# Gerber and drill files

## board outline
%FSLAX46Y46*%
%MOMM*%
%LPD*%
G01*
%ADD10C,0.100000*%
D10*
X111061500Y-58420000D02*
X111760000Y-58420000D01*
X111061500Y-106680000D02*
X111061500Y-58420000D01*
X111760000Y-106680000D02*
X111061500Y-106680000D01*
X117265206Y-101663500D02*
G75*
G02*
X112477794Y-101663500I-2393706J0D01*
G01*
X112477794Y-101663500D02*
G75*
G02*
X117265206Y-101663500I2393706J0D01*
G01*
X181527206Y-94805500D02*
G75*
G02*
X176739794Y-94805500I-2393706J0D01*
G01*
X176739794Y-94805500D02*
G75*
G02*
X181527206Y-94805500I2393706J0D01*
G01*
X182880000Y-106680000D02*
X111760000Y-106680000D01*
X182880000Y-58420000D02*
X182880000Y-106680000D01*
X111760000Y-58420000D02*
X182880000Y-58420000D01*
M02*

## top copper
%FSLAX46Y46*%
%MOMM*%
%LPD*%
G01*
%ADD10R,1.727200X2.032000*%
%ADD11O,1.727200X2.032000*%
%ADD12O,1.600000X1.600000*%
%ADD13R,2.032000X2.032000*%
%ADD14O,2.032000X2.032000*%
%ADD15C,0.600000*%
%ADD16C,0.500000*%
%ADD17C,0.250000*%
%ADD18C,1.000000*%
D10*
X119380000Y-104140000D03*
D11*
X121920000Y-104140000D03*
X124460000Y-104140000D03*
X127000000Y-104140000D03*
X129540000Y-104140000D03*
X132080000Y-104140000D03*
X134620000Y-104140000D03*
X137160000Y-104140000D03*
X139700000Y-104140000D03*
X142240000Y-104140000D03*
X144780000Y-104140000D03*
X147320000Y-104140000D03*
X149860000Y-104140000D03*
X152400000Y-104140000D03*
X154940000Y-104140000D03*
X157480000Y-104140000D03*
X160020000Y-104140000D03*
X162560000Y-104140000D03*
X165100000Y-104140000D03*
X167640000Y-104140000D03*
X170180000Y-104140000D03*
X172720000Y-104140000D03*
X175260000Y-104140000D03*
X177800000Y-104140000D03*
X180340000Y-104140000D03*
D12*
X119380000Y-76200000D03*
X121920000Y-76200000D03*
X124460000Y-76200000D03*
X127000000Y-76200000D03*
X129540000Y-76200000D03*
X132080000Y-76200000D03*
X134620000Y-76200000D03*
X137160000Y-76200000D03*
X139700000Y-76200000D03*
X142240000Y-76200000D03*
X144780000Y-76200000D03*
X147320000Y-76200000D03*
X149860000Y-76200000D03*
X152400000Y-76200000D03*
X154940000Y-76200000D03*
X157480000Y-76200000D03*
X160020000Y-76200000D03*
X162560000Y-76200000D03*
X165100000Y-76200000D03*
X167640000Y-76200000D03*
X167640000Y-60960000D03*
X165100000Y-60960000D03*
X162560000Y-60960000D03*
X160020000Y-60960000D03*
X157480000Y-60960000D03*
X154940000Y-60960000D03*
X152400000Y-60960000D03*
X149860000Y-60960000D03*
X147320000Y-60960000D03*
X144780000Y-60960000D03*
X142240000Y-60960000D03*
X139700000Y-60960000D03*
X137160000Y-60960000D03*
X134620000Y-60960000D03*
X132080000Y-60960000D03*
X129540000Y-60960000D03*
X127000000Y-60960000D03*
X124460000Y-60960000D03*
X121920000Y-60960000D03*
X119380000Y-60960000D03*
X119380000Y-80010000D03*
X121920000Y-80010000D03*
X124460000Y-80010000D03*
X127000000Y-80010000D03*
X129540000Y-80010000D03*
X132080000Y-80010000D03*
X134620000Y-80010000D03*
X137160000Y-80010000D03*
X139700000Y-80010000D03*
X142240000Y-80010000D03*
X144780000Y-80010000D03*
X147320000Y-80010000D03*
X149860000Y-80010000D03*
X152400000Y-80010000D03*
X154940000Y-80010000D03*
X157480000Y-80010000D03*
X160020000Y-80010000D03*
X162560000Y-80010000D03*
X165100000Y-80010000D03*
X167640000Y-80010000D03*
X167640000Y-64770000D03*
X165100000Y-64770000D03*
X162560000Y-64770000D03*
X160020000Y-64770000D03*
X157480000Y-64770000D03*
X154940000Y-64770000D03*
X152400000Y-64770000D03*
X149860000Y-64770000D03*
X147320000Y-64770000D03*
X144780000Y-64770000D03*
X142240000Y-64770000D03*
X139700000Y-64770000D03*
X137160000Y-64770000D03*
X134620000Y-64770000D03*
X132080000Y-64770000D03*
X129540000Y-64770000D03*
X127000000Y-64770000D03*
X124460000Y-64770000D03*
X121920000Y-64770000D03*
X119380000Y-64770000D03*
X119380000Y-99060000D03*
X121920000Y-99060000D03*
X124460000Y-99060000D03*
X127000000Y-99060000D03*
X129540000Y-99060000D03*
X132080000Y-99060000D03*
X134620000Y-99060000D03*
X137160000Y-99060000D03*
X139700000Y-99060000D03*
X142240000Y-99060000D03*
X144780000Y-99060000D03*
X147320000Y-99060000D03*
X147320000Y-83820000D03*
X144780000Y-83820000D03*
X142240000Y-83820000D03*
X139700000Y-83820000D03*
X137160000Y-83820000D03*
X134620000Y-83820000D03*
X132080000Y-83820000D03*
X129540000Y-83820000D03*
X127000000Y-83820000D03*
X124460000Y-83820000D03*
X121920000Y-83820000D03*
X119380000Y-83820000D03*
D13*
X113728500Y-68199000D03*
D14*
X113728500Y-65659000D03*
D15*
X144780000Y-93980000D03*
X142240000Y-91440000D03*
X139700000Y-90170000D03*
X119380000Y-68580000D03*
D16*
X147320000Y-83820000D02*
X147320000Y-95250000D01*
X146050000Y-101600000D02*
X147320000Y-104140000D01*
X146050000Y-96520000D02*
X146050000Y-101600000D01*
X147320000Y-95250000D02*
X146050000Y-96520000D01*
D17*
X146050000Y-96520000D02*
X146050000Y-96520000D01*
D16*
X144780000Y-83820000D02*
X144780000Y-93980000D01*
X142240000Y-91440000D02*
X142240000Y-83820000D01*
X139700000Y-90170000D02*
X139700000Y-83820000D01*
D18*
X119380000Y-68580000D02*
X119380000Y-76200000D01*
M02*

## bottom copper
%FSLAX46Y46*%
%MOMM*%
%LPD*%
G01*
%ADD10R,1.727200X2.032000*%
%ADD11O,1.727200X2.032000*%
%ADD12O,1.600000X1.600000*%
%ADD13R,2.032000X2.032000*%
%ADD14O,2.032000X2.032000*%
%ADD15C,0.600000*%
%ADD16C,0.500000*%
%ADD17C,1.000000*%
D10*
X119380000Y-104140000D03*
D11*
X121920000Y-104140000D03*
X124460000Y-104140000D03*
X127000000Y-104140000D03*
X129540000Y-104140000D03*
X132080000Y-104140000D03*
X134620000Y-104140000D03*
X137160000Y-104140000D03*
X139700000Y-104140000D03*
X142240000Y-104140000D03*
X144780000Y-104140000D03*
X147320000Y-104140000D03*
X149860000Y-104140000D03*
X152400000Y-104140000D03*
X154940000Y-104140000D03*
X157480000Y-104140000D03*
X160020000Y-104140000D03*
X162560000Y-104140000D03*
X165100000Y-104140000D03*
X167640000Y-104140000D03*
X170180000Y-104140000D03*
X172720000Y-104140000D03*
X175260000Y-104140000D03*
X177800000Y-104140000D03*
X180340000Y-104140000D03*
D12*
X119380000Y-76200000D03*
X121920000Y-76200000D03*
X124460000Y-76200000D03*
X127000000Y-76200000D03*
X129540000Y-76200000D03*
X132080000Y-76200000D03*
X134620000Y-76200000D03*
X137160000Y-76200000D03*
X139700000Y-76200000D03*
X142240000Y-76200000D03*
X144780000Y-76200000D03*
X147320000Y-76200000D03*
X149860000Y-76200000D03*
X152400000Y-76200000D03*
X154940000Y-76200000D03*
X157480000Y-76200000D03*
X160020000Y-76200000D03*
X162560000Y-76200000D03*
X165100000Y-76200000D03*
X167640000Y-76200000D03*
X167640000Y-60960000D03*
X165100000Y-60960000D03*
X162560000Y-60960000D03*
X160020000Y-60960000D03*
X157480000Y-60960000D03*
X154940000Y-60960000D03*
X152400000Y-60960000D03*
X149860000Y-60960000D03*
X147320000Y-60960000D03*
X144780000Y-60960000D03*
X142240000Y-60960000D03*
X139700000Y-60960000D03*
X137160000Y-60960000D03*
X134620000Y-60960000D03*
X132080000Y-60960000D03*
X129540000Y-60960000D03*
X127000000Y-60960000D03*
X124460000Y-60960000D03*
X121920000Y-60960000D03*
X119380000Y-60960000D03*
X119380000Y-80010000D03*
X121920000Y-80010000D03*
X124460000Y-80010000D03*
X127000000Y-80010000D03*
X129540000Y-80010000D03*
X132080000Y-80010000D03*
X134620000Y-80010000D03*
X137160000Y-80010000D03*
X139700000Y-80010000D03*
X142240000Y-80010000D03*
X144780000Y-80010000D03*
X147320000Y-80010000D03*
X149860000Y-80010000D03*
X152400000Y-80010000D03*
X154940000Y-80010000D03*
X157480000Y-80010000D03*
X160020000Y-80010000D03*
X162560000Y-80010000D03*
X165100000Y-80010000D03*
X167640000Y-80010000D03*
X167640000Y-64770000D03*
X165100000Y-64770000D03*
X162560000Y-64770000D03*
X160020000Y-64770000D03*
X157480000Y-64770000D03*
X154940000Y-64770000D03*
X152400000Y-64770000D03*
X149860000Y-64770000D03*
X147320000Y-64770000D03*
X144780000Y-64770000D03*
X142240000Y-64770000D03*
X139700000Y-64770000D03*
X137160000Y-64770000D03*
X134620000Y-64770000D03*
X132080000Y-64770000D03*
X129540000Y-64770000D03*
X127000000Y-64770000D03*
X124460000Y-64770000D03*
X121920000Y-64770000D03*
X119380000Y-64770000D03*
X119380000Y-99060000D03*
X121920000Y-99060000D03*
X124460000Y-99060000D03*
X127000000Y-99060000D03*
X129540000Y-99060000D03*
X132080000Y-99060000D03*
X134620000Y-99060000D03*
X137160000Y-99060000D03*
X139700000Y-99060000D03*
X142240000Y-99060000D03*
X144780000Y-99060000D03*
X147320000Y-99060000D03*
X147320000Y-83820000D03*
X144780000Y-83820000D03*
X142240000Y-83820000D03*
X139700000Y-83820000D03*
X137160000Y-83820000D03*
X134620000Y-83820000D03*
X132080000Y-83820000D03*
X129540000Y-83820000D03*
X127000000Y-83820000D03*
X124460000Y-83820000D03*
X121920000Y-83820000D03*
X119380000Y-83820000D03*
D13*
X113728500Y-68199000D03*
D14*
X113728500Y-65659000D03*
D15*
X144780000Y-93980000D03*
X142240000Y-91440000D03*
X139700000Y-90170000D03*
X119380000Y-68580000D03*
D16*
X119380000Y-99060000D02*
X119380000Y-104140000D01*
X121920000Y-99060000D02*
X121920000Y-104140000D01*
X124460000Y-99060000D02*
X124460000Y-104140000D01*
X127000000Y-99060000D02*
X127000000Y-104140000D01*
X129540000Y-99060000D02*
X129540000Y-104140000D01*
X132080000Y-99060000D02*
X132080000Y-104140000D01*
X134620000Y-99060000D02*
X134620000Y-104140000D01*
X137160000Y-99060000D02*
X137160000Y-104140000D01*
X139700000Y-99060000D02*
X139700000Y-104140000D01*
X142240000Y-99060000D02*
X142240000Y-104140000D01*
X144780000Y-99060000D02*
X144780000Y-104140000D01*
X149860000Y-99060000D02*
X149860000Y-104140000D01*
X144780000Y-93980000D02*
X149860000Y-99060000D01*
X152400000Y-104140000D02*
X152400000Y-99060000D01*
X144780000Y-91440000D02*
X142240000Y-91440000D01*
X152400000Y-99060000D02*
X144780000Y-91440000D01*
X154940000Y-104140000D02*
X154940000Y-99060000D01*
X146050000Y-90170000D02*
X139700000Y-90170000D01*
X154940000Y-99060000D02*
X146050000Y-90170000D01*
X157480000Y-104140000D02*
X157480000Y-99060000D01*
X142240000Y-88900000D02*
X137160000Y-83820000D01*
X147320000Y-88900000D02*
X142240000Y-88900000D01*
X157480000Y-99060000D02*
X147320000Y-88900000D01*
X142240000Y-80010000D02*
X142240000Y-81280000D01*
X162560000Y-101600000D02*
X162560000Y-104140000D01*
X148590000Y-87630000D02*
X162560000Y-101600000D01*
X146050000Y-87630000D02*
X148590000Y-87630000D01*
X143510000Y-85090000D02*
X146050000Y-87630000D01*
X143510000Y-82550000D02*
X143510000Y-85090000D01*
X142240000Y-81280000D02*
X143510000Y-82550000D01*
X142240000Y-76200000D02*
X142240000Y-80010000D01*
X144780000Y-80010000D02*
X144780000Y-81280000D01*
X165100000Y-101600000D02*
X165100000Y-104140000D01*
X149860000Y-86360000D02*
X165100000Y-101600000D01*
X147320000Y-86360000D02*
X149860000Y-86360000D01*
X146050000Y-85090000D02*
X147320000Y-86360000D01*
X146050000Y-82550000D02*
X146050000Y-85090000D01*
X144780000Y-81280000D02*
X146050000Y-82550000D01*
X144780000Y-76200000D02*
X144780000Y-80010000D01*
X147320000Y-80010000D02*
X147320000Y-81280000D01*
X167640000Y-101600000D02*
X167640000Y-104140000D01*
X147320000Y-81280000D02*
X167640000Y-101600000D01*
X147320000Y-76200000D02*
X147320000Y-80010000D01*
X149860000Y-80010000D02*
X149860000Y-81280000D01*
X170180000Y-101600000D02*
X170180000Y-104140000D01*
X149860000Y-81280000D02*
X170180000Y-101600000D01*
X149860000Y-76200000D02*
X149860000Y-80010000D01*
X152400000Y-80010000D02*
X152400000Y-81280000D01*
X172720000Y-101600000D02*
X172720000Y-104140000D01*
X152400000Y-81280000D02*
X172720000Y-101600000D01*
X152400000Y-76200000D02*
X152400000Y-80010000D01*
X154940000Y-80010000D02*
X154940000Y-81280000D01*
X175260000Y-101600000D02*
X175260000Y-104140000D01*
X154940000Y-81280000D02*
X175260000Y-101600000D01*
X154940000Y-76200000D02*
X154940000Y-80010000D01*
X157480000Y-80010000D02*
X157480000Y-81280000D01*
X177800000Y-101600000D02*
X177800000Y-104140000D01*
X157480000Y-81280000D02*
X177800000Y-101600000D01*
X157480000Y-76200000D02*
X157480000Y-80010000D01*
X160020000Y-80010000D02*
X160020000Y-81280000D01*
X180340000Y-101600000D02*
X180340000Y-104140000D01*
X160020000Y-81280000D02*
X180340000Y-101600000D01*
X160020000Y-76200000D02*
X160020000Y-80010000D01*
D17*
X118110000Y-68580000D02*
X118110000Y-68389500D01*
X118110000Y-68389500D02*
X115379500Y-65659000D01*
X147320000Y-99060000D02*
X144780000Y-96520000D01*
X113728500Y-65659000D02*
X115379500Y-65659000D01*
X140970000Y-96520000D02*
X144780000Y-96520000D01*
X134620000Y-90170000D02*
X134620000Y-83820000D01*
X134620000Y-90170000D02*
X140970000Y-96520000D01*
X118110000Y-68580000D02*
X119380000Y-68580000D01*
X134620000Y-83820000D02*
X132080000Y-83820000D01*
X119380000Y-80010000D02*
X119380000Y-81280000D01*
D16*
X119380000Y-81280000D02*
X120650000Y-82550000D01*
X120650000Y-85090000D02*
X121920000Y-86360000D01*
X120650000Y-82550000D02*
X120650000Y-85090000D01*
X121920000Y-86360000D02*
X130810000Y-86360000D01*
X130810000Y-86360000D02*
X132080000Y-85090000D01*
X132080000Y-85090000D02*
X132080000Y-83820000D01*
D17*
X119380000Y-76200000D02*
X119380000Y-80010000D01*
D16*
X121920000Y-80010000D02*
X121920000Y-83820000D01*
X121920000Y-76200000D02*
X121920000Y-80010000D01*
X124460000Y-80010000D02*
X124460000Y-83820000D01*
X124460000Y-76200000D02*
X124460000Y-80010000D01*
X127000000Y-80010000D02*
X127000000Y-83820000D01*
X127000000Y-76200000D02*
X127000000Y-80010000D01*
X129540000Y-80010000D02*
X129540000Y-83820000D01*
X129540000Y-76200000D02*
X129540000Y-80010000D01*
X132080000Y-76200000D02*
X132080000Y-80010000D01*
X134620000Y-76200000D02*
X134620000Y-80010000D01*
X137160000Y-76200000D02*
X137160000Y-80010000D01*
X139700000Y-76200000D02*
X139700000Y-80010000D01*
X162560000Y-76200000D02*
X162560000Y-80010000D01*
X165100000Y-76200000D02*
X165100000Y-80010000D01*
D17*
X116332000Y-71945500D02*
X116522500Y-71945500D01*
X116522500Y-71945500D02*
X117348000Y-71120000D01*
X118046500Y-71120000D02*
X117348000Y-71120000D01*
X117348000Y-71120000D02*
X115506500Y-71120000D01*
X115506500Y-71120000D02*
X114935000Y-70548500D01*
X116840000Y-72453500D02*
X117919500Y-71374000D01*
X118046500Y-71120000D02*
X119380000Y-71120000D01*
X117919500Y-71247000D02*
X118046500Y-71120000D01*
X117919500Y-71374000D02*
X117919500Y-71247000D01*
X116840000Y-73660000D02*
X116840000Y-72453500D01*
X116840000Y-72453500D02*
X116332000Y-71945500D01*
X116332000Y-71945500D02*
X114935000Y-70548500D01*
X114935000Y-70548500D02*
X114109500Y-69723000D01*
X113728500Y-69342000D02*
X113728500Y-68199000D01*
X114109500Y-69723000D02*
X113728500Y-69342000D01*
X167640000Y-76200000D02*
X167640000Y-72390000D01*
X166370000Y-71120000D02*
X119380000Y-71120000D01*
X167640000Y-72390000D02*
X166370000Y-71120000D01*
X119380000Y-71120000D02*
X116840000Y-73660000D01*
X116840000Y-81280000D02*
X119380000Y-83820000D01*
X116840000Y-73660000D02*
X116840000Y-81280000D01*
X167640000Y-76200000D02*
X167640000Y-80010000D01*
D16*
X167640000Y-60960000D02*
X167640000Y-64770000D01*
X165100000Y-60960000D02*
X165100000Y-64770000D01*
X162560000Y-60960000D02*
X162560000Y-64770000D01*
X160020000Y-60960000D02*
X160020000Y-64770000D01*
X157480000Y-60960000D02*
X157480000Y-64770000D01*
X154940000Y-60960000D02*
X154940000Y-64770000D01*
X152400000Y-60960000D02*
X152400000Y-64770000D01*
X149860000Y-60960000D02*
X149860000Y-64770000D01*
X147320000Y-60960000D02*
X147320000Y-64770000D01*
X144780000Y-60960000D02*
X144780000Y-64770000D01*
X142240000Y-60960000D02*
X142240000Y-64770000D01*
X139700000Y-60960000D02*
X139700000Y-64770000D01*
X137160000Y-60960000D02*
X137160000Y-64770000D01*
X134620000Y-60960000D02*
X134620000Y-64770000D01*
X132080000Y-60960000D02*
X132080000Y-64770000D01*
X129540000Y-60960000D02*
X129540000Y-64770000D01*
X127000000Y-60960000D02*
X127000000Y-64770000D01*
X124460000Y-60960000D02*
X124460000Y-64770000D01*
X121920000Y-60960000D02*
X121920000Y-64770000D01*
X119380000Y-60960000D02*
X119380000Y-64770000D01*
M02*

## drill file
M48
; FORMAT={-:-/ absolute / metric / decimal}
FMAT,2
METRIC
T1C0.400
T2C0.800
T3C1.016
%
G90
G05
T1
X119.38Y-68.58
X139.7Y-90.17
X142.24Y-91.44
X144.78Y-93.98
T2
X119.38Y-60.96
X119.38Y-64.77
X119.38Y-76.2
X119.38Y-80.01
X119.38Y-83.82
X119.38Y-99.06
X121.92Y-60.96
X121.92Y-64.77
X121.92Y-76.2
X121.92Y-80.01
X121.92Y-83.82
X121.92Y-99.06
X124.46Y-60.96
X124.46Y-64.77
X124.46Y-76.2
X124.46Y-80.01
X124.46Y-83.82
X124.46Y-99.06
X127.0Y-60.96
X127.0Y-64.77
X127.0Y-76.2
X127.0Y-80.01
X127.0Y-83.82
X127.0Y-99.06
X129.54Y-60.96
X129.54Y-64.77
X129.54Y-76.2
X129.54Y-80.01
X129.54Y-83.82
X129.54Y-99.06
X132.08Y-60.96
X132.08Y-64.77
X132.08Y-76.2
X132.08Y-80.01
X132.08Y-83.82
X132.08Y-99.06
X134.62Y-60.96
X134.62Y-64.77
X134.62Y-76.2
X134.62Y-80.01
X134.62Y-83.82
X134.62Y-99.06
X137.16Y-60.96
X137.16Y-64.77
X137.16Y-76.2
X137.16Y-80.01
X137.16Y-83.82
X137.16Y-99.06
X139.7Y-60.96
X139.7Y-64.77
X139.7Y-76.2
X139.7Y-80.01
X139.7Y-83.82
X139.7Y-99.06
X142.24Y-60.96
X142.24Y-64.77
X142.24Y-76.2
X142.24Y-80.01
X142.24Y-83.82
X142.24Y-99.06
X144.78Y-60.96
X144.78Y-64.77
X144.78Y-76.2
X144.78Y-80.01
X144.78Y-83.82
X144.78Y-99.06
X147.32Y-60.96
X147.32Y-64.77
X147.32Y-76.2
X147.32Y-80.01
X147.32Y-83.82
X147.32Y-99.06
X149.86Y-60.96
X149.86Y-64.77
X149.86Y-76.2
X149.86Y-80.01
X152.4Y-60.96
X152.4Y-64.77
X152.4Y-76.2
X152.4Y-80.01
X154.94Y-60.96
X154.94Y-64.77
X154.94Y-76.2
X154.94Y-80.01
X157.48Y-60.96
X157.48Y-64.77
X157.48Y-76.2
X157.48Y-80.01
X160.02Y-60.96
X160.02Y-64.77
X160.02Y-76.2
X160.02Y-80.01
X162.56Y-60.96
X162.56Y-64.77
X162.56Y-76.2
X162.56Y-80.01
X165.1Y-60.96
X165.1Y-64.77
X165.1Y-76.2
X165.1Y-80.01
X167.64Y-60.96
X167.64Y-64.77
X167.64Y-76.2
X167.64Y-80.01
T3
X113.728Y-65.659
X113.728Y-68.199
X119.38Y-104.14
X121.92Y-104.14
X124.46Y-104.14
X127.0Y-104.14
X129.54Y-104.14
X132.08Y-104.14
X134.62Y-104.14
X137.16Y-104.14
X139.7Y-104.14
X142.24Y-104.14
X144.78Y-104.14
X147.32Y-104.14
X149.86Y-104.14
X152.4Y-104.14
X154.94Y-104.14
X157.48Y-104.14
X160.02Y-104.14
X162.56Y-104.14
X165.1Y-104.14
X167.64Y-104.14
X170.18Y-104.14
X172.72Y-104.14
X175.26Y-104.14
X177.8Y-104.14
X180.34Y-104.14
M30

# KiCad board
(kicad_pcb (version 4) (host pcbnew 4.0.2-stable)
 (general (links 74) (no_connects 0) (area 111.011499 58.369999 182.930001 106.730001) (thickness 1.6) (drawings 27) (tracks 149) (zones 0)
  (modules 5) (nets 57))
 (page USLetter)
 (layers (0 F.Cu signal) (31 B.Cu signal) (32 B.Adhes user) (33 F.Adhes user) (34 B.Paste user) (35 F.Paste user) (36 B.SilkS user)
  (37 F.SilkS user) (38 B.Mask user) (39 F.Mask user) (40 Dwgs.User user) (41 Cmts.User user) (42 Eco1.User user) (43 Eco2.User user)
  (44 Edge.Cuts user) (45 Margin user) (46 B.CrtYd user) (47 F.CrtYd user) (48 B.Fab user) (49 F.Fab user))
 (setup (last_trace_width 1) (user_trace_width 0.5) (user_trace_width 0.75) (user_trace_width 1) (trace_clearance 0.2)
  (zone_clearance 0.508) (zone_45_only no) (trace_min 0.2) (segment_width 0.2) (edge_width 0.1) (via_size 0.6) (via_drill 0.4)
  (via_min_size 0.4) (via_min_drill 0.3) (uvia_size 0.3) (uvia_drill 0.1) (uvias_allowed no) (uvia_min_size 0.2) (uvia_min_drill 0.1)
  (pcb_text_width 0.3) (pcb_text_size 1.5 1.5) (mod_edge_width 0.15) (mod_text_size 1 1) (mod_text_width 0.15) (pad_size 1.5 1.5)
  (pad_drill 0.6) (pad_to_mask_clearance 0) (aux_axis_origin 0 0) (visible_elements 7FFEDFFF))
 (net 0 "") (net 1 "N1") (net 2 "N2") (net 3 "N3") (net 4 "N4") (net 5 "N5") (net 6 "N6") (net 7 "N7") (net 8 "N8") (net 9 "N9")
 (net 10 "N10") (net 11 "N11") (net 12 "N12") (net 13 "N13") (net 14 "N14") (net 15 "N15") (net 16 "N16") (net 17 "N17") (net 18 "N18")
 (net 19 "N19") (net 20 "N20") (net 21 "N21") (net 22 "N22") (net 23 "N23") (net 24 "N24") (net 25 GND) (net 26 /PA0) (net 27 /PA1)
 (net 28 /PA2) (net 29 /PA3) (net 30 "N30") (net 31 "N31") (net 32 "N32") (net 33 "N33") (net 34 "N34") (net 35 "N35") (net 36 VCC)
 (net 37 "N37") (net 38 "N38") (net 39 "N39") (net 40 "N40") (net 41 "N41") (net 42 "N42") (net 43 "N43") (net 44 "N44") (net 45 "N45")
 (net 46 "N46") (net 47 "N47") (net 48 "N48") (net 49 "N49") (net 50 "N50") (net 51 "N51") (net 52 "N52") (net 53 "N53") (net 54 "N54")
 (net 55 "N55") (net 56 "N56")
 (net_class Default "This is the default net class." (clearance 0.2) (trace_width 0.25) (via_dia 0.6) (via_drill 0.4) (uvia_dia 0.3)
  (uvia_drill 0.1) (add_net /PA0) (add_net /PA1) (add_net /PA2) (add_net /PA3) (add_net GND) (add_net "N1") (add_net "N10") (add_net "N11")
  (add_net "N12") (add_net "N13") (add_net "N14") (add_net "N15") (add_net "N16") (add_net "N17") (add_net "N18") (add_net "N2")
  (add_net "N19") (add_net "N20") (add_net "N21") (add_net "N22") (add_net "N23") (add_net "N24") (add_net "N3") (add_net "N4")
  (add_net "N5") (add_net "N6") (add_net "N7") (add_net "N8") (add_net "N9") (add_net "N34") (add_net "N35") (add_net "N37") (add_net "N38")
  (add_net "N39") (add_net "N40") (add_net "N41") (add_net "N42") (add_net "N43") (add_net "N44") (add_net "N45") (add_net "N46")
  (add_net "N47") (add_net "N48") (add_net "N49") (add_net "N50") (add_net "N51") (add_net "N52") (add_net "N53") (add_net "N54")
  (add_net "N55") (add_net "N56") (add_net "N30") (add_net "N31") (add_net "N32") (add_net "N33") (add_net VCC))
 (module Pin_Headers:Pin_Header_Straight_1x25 (layer F.Cu) (at 119.38 104.14 90)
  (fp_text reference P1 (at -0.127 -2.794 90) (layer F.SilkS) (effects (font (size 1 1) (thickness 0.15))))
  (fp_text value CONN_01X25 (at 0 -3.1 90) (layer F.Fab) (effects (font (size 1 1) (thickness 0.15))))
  (pad 1 thru_hole rect (at 0 0 90) (size 2.032 1.7272) (drill 1.016) (layers *.Cu *.Mask F.SilkS) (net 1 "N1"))
  (pad 2 thru_hole oval (at 0 2.54 90) (size 2.032 1.7272) (drill 1.016) (layers *.Cu *.Mask F.SilkS) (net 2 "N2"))
  (pad 3 thru_hole oval (at 0 5.08 90) (size 2.032 1.7272) (drill 1.016) (layers *.Cu *.Mask F.SilkS) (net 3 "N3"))
  (pad 4 thru_hole oval (at 0 7.62 90) (size 2.032 1.7272) (drill 1.016) (layers *.Cu *.Mask F.SilkS) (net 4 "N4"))
  (pad 5 thru_hole oval (at 0 10.16 90) (size 2.032 1.7272) (drill 1.016) (layers *.Cu *.Mask F.SilkS) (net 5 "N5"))
  (pad 6 thru_hole oval (at 0 12.7 90) (size 2.032 1.7272) (drill 1.016) (layers *.Cu *.Mask F.SilkS) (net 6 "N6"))
  (pad 7 thru_hole oval (at 0 15.24 90) (size 2.032 1.7272) (drill 1.016) (layers *.Cu *.Mask F.SilkS) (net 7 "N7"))
  (pad 8 thru_hole oval (at 0 17.78 90) (size 2.032 1.7272) (drill 1.016) (layers *.Cu *.Mask F.SilkS) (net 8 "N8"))
  (pad 9 thru_hole oval (at 0 20.32 90) (size 2.032 1.7272) (drill 1.016) (layers *.Cu *.Mask F.SilkS) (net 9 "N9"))
  (pad 10 thru_hole oval (at 0 22.86 90) (size 2.032 1.7272) (drill 1.016) (layers *.Cu *.Mask F.SilkS) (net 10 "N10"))
  (pad 11 thru_hole oval (at 0 25.4 90) (size 2.032 1.7272) (drill 1.016) (layers *.Cu *.Mask F.SilkS) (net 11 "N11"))
  (pad 12 thru_hole oval (at 0 27.94 90) (size 2.032 1.7272) (drill 1.016) (layers *.Cu *.Mask F.SilkS) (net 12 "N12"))
  (pad 13 thru_hole oval (at 0 30.48 90) (size 2.032 1.7272) (drill 1.016) (layers *.Cu *.Mask F.SilkS) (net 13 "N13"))
  (pad 14 thru_hole oval (at 0 33.02 90) (size 2.032 1.7272) (drill 1.016) (layers *.Cu *.Mask F.SilkS) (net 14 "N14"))
  (pad 15 thru_hole oval (at 0 35.56 90) (size 2.032 1.7272) (drill 1.016) (layers *.Cu *.Mask F.SilkS) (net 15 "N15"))
  (pad 16 thru_hole oval (at 0 38.1 90) (size 2.032 1.7272) (drill 1.016) (layers *.Cu *.Mask F.SilkS) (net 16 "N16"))
  (pad 17 thru_hole oval (at 0 40.64 90) (size 2.032 1.7272) (drill 1.016) (layers *.Cu *.Mask F.SilkS))
  (pad 18 thru_hole oval (at 0 43.18 90) (size 2.032 1.7272) (drill 1.016) (layers *.Cu *.Mask F.SilkS) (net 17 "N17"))
  (pad 19 thru_hole oval (at 0 45.72 90) (size 2.032 1.7272) (drill 1.016) (layers *.Cu *.Mask F.SilkS) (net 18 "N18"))
  (pad 20 thru_hole oval (at 0 48.26 90) (size 2.032 1.7272) (drill 1.016) (layers *.Cu *.Mask F.SilkS) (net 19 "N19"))
  (pad 21 thru_hole oval (at 0 50.8 90) (size 2.032 1.7272) (drill 1.016) (layers *.Cu *.Mask F.SilkS) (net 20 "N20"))
  (pad 22 thru_hole oval (at 0 53.34 90) (size 2.032 1.7272) (drill 1.016) (layers *.Cu *.Mask F.SilkS) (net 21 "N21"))
  (pad 23 thru_hole oval (at 0 55.88 90) (size 2.032 1.7272) (drill 1.016) (layers *.Cu *.Mask F.SilkS) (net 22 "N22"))
  (pad 24 thru_hole oval (at 0 58.42 90) (size 2.032 1.7272) (drill 1.016) (layers *.Cu *.Mask F.SilkS) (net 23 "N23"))
  (pad 25 thru_hole oval (at 0 60.96 90) (size 2.032 1.7272) (drill 1.016) (layers *.Cu *.Mask F.SilkS) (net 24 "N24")))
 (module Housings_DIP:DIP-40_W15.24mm (layer F.Cu) (at 119.38 76.2 90)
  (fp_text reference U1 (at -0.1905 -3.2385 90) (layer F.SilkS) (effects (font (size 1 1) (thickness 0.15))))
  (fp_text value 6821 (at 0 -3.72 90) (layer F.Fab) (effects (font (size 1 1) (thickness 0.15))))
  (pad 1 thru_hole oval (at 0 0 90) (size 1.6 1.6) (drill 0.8) (layers *.Cu *.Mask F.SilkS) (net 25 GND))
  (pad 2 thru_hole oval (at 0 2.54 90) (size 1.6 1.6) (drill 0.8) (layers *.Cu *.Mask F.SilkS) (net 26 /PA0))
  (pad 3 thru_hole oval (at 0 5.08 90) (size 1.6 1.6) (drill 0.8) (layers *.Cu *.Mask F.SilkS) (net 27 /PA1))
  (pad 4 thru_hole oval (at 0 7.62 90) (size 1.6 1.6) (drill 0.8) (layers *.Cu *.Mask F.SilkS) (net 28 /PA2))
  (pad 5 thru_hole oval (at 0 10.16 90) (size 1.6 1.6) (drill 0.8) (layers *.Cu *.Mask F.SilkS) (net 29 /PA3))
  (pad 6 thru_hole oval (at 0 12.7 90) (size 1.6 1.6) (drill 0.8) (layers *.Cu *.Mask F.SilkS) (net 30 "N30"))
  (pad 7 thru_hole oval (at 0 15.24 90) (size 1.6 1.6) (drill 0.8) (layers *.Cu *.Mask F.SilkS) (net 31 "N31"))
  (pad 8 thru_hole oval (at 0 17.78 90) (size 1.6 1.6) (drill 0.8) (layers *.Cu *.Mask F.SilkS) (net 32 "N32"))
  (pad 9 thru_hole oval (at 0 20.32 90) (size 1.6 1.6) (drill 0.8) (layers *.Cu *.Mask F.SilkS) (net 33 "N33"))
  (pad 10 thru_hole oval (at 0 22.86 90) (size 1.6 1.6) (drill 0.8) (layers *.Cu *.Mask F.SilkS) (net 17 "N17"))
  (pad 11 thru_hole oval (at 0 25.4 90) (size 1.6 1.6) (drill 0.8) (layers *.Cu *.Mask F.SilkS) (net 18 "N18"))
  (pad 12 thru_hole oval (at 0 27.94 90) (size 1.6 1.6) (drill 0.8) (layers *.Cu *.Mask F.SilkS) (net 19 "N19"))
  (pad 13 thru_hole oval (at 0 30.48 90) (size 1.6 1.6) (drill 0.8) (layers *.Cu *.Mask F.SilkS) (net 20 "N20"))
  (pad 14 thru_hole oval (at 0 33.02 90) (size 1.6 1.6) (drill 0.8) (layers *.Cu *.Mask F.SilkS) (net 21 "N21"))
  (pad 15 thru_hole oval (at 0 35.56 90) (size 1.6 1.6) (drill 0.8) (layers *.Cu *.Mask F.SilkS) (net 22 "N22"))
  (pad 16 thru_hole oval (at 0 38.1 90) (size 1.6 1.6) (drill 0.8) (layers *.Cu *.Mask F.SilkS) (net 23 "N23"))
  (pad 17 thru_hole oval (at 0 40.64 90) (size 1.6 1.6) (drill 0.8) (layers *.Cu *.Mask F.SilkS) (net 24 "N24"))
  (pad 18 thru_hole oval (at 0 43.18 90) (size 1.6 1.6) (drill 0.8) (layers *.Cu *.Mask F.SilkS) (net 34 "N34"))
  (pad 19 thru_hole oval (at 0 45.72 90) (size 1.6 1.6) (drill 0.8) (layers *.Cu *.Mask F.SilkS) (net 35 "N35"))
  (pad 20 thru_hole oval (at 0 48.26 90) (size 1.6 1.6) (drill 0.8) (layers *.Cu *.Mask F.SilkS) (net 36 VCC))
  (pad 21 thru_hole oval (at 15.24 48.26 90) (size 1.6 1.6) (drill 0.8) (layers *.Cu *.Mask F.SilkS) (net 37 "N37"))
  (pad 22 thru_hole oval (at 15.24 45.72 90) (size 1.6 1.6) (drill 0.8) (layers *.Cu *.Mask F.SilkS) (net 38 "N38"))
  (pad 23 thru_hole oval (at 15.24 43.18 90) (size 1.6 1.6) (drill 0.8) (layers *.Cu *.Mask F.SilkS) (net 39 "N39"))
  (pad 24 thru_hole oval (at 15.24 40.64 90) (size 1.6 1.6) (drill 0.8) (layers *.Cu *.Mask F.SilkS) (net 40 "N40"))
  (pad 25 thru_hole oval (at 15.24 38.1 90) (size 1.6 1.6) (drill 0.8) (layers *.Cu *.Mask F.SilkS) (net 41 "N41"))
  (pad 26 thru_hole oval (at 15.24 35.56 90) (size 1.6 1.6) (drill 0.8) (layers *.Cu *.Mask F.SilkS) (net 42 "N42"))
  (pad 27 thru_hole oval (at 15.24 33.02 90) (size 1.6 1.6) (drill 0.8) (layers *.Cu *.Mask F.SilkS) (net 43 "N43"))
  (pad 28 thru_hole oval (at 15.24 30.48 90) (size 1.6 1.6) (drill 0.8) (layers *.Cu *.Mask F.SilkS) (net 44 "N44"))
  (pad 29 thru_hole oval (at 15.24 27.94 90) (size 1.6 1.6) (drill 0.8) (layers *.Cu *.Mask F.SilkS) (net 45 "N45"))
  (pad 30 thru_hole oval (at 15.24 25.4 90) (size 1.6 1.6) (drill 0.8) (layers *.Cu *.Mask F.SilkS) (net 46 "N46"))
  (pad 31 thru_hole oval (at 15.24 22.86 90) (size 1.6 1.6) (drill 0.8) (layers *.Cu *.Mask F.SilkS) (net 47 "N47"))
  (pad 32 thru_hole oval (at 15.24 20.32 90) (size 1.6 1.6) (drill 0.8) (layers *.Cu *.Mask F.SilkS) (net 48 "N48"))
  (pad 33 thru_hole oval (at 15.24 17.78 90) (size 1.6 1.6) (drill 0.8) (layers *.Cu *.Mask F.SilkS) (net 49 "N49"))
  (pad 34 thru_hole oval (at 15.24 15.24 90) (size 1.6 1.6) (drill 0.8) (layers *.Cu *.Mask F.SilkS) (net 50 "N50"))
  (pad 35 thru_hole oval (at 15.24 12.7 90) (size 1.6 1.6) (drill 0.8) (layers *.Cu *.Mask F.SilkS) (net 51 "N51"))
  (pad 36 thru_hole oval (at 15.24 10.16 90) (size 1.6 1.6) (drill 0.8) (layers *.Cu *.Mask F.SilkS) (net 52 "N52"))
  (pad 37 thru_hole oval (at 15.24 7.62 90) (size 1.6 1.6) (drill 0.8) (layers *.Cu *.Mask F.SilkS) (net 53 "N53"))
  (pad 38 thru_hole oval (at 15.24 5.08 90) (size 1.6 1.6) (drill 0.8) (layers *.Cu *.Mask F.SilkS) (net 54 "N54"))
  (pad 39 thru_hole oval (at 15.24 2.54 90) (size 1.6 1.6) (drill 0.8) (layers *.Cu *.Mask F.SilkS) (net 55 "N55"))
  (pad 40 thru_hole oval (at 15.24 0 90) (size 1.6 1.6) (drill 0.8) (layers *.Cu *.Mask F.SilkS) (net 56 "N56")))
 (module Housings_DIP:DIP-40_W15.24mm (layer F.Cu) (at 119.38 80.01 90)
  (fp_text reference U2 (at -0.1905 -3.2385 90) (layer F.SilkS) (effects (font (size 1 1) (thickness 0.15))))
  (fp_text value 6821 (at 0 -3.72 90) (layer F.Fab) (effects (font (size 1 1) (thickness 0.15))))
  (pad 1 thru_hole oval (at 0 0 90) (size 1.6 1.6) (drill 0.8) (layers *.Cu *.Mask F.SilkS) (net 25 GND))
  (pad 2 thru_hole oval (at 0 2.54 90) (size 1.6 1.6) (drill 0.8) (layers *.Cu *.Mask F.SilkS) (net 26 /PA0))
  (pad 3 thru_hole oval (at 0 5.08 90) (size 1.6 1.6) (drill 0.8) (layers *.Cu *.Mask F.SilkS) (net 27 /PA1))
  (pad 4 thru_hole oval (at 0 7.62 90) (size 1.6 1.6) (drill 0.8) (layers *.Cu *.Mask F.SilkS) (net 28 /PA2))
  (pad 5 thru_hole oval (at 0 10.16 90) (size 1.6 1.6) (drill 0.8) (layers *.Cu *.Mask F.SilkS) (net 29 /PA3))
  (pad 6 thru_hole oval (at 0 12.7 90) (size 1.6 1.6) (drill 0.8) (layers *.Cu *.Mask F.SilkS) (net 30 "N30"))
  (pad 7 thru_hole oval (at 0 15.24 90) (size 1.6 1.6) (drill 0.8) (layers *.Cu *.Mask F.SilkS) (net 31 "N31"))
  (pad 8 thru_hole oval (at 0 17.78 90) (size 1.6 1.6) (drill 0.8) (layers *.Cu *.Mask F.SilkS) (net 32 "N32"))
  (pad 9 thru_hole oval (at 0 20.32 90) (size 1.6 1.6) (drill 0.8) (layers *.Cu *.Mask F.SilkS) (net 33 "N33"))
  (pad 10 thru_hole oval (at 0 22.86 90) (size 1.6 1.6) (drill 0.8) (layers *.Cu *.Mask F.SilkS) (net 17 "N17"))
  (pad 11 thru_hole oval (at 0 25.4 90) (size 1.6 1.6) (drill 0.8) (layers *.Cu *.Mask F.SilkS) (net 18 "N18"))
  (pad 12 thru_hole oval (at 0 27.94 90) (size 1.6 1.6) (drill 0.8) (layers *.Cu *.Mask F.SilkS) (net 19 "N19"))
  (pad 13 thru_hole oval (at 0 30.48 90) (size 1.6 1.6) (drill 0.8) (layers *.Cu *.Mask F.SilkS) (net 20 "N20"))
  (pad 14 thru_hole oval (at 0 33.02 90) (size 1.6 1.6) (drill 0.8) (layers *.Cu *.Mask F.SilkS) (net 21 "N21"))
  (pad 15 thru_hole oval (at 0 35.56 90) (size 1.6 1.6) (drill 0.8) (layers *.Cu *.Mask F.SilkS) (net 22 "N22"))
  (pad 16 thru_hole oval (at 0 38.1 90) (size 1.6 1.6) (drill 0.8) (layers *.Cu *.Mask F.SilkS) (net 23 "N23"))
  (pad 17 thru_hole oval (at 0 40.64 90) (size 1.6 1.6) (drill 0.8) (layers *.Cu *.Mask F.SilkS) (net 24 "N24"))
  (pad 18 thru_hole oval (at 0 43.18 90) (size 1.6 1.6) (drill 0.8) (layers *.Cu *.Mask F.SilkS) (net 34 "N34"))
  (pad 19 thru_hole oval (at 0 45.72 90) (size 1.6 1.6) (drill 0.8) (layers *.Cu *.Mask F.SilkS) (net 35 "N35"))
  (pad 20 thru_hole oval (at 0 48.26 90) (size 1.6 1.6) (drill 0.8) (layers *.Cu *.Mask F.SilkS) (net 36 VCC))
  (pad 21 thru_hole oval (at 15.24 48.26 90) (size 1.6 1.6) (drill 0.8) (layers *.Cu *.Mask F.SilkS) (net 37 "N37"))
  (pad 22 thru_hole oval (at 15.24 45.72 90) (size 1.6 1.6) (drill 0.8) (layers *.Cu *.Mask F.SilkS) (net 38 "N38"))
  (pad 23 thru_hole oval (at 15.24 43.18 90) (size 1.6 1.6) (drill 0.8) (layers *.Cu *.Mask F.SilkS) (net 39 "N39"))
  (pad 24 thru_hole oval (at 15.24 40.64 90) (size 1.6 1.6) (drill 0.8) (layers *.Cu *.Mask F.SilkS) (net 40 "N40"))
  (pad 25 thru_hole oval (at 15.24 38.1 90) (size 1.6 1.6) (drill 0.8) (layers *.Cu *.Mask F.SilkS) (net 41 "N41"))
  (pad 26 thru_hole oval (at 15.24 35.56 90) (size 1.6 1.6) (drill 0.8) (layers *.Cu *.Mask F.SilkS) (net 42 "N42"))
  (pad 27 thru_hole oval (at 15.24 33.02 90) (size 1.6 1.6) (drill 0.8) (layers *.Cu *.Mask F.SilkS) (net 43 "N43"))
  (pad 28 thru_hole oval (at 15.24 30.48 90) (size 1.6 1.6) (drill 0.8) (layers *.Cu *.Mask F.SilkS) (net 44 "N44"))
  (pad 29 thru_hole oval (at 15.24 27.94 90) (size 1.6 1.6) (drill 0.8) (layers *.Cu *.Mask F.SilkS) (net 45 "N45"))
  (pad 30 thru_hole oval (at 15.24 25.4 90) (size 1.6 1.6) (drill 0.8) (layers *.Cu *.Mask F.SilkS) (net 46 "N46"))
  (pad 31 thru_hole oval (at 15.24 22.86 90) (size 1.6 1.6) (drill 0.8) (layers *.Cu *.Mask F.SilkS) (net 47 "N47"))
  (pad 32 thru_hole oval (at 15.24 20.32 90) (size 1.6 1.6) (drill 0.8) (layers *.Cu *.Mask F.SilkS) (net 48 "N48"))
  (pad 33 thru_hole oval (at 15.24 17.78 90) (size 1.6 1.6) (drill 0.8) (layers *.Cu *.Mask F.SilkS) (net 49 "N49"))
  (pad 34 thru_hole oval (at 15.24 15.24 90) (size 1.6 1.6) (drill 0.8) (layers *.Cu *.Mask F.SilkS) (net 50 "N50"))
  (pad 35 thru_hole oval (at 15.24 12.7 90) (size 1.6 1.6) (drill 0.8) (layers *.Cu *.Mask F.SilkS) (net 51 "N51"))
  (pad 36 thru_hole oval (at 15.24 10.16 90) (size 1.6 1.6) (drill 0.8) (layers *.Cu *.Mask F.SilkS) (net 52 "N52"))
  (pad 37 thru_hole oval (at 15.24 7.62 90) (size 1.6 1.6) (drill 0.8) (layers *.Cu *.Mask F.SilkS) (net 53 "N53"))
  (pad 38 thru_hole oval (at 15.24 5.08 90) (size 1.6 1.6) (drill 0.8) (layers *.Cu *.Mask F.SilkS) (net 54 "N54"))
  (pad 39 thru_hole oval (at 15.24 2.54 90) (size 1.6 1.6) (drill 0.8) (layers *.Cu *.Mask F.SilkS) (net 55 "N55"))
  (pad 40 thru_hole oval (at 15.24 0 90) (size 1.6 1.6) (drill 0.8) (layers *.Cu *.Mask F.SilkS) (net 56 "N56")))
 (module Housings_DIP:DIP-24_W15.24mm (layer F.Cu) (at 119.38 99.06 90)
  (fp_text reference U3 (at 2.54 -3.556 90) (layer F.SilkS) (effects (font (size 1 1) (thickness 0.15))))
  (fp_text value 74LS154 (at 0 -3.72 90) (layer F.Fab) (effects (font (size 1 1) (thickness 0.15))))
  (pad 1 thru_hole oval (at 0 0 90) (size 1.6 1.6) (drill 0.8) (layers *.Cu *.Mask F.SilkS) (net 1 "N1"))
  (pad 2 thru_hole oval (at 0 2.54 90) (size 1.6 1.6) (drill 0.8) (layers *.Cu *.Mask F.SilkS) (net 2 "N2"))
  (pad 3 thru_hole oval (at 0 5.08 90) (size 1.6 1.6) (drill 0.8) (layers *.Cu *.Mask F.SilkS) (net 3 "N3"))
  (pad 4 thru_hole oval (at 0 7.62 90) (size 1.6 1.6) (drill 0.8) (layers *.Cu *.Mask F.SilkS) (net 4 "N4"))
  (pad 5 thru_hole oval (at 0 10.16 90) (size 1.6 1.6) (drill 0.8) (layers *.Cu *.Mask F.SilkS) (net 5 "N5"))
  (pad 6 thru_hole oval (at 0 12.7 90) (size 1.6 1.6) (drill 0.8) (layers *.Cu *.Mask F.SilkS) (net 6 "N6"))
  (pad 7 thru_hole oval (at 0 15.24 90) (size 1.6 1.6) (drill 0.8) (layers *.Cu *.Mask F.SilkS) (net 7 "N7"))
  (pad 8 thru_hole oval (at 0 17.78 90) (size 1.6 1.6) (drill 0.8) (layers *.Cu *.Mask F.SilkS) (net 8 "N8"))
  (pad 9 thru_hole oval (at 0 20.32 90) (size 1.6 1.6) (drill 0.8) (layers *.Cu *.Mask F.SilkS) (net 9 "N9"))
  (pad 10 thru_hole oval (at 0 22.86 90) (size 1.6 1.6) (drill 0.8) (layers *.Cu *.Mask F.SilkS) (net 10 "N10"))
  (pad 11 thru_hole oval (at 0 25.4 90) (size 1.6 1.6) (drill 0.8) (layers *.Cu *.Mask F.SilkS) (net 11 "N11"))
  (pad 12 thru_hole oval (at 0 27.94 90) (size 1.6 1.6) (drill 0.8) (layers *.Cu *.Mask F.SilkS) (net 25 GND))
  (pad 13 thru_hole oval (at 15.24 27.94 90) (size 1.6 1.6) (drill 0.8) (layers *.Cu *.Mask F.SilkS) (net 12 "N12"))
  (pad 14 thru_hole oval (at 15.24 25.4 90) (size 1.6 1.6) (drill 0.8) (layers *.Cu *.Mask F.SilkS) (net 13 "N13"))
  (pad 15 thru_hole oval (at 15.24 22.86 90) (size 1.6 1.6) (drill 0.8) (layers *.Cu *.Mask F.SilkS) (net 14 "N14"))
  (pad 16 thru_hole oval (at 15.24 20.32 90) (size 1.6 1.6) (drill 0.8) (layers *.Cu *.Mask F.SilkS) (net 15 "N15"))
  (pad 17 thru_hole oval (at 15.24 17.78 90) (size 1.6 1.6) (drill 0.8) (layers *.Cu *.Mask F.SilkS) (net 16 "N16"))
  (pad 18 thru_hole oval (at 15.24 15.24 90) (size 1.6 1.6) (drill 0.8) (layers *.Cu *.Mask F.SilkS) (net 25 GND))
  (pad 19 thru_hole oval (at 15.24 12.7 90) (size 1.6 1.6) (drill 0.8) (layers *.Cu *.Mask F.SilkS) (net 25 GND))
  (pad 20 thru_hole oval (at 15.24 10.16 90) (size 1.6 1.6) (drill 0.8) (layers *.Cu *.Mask F.SilkS) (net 29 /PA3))
  (pad 21 thru_hole oval (at 15.24 7.62 90) (size 1.6 1.6) (drill 0.8) (layers *.Cu *.Mask F.SilkS) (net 28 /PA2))
  (pad 22 thru_hole oval (at 15.24 5.08 90) (size 1.6 1.6) (drill 0.8) (layers *.Cu *.Mask F.SilkS) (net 27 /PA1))
  (pad 23 thru_hole oval (at 15.24 2.54 90) (size 1.6 1.6) (drill 0.8) (layers *.Cu *.Mask F.SilkS) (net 26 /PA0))
  (pad 24 thru_hole oval (at 15.24 0 90) (size 1.6 1.6) (drill 0.8) (layers *.Cu *.Mask F.SilkS) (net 36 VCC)))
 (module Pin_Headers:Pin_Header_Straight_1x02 (layer F.Cu) (at 113.7285 68.199 180)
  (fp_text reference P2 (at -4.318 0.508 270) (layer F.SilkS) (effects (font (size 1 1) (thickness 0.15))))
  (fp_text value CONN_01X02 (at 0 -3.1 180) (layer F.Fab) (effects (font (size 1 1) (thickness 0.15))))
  (pad 1 thru_hole rect (at 0 0 180) (size 2.032 2.032) (drill 1.016) (layers *.Cu *.Mask F.SilkS) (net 36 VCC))
  (pad 2 thru_hole oval (at 0 2.54 180) (size 2.032 2.032) (drill 1.016) (layers *.Cu *.Mask F.SilkS) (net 25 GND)))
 (gr_line (start 111.0615 58.42) (end 111.76 58.42) (angle 90) (layer Edge.Cuts) (width 0.1))
 (gr_line (start 111.0615 106.68) (end 111.0615 58.42) (angle 90) (layer Edge.Cuts) (width 0.1))
 (gr_line (start 111.76 106.68) (end 111.0615 106.68) (angle 90) (layer Edge.Cuts) (width 0.1))
 (gr_circle (center 114.8715 101.6635) (end 117.094 102.5525) (layer Edge.Cuts) (width 0.1))
 (gr_circle (center 179.1335 94.8055) (end 181.356 95.6945) (layer Edge.Cuts) (width 0.1))
 (gr_line (start 182.88 106.68) (end 111.76 106.68) (angle 90) (layer Edge.Cuts) (width 0.1))
 (gr_line (start 182.88 58.42) (end 182.88 106.68) (angle 90) (layer Edge.Cuts) (width 0.1))
 (gr_line (start 111.76 58.42) (end 182.88 58.42) (angle 90) (layer Edge.Cuts) (width 0.1))
 (segment (start 119.38 99.06) (end 119.38 104.14) (width 0.5) (layer B.Cu) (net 1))
 (segment (start 121.92 99.06) (end 121.92 104.14) (width 0.5) (layer B.Cu) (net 2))
 (segment (start 124.46 99.06) (end 124.46 104.14) (width 0.5) (layer B.Cu) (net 3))
 (segment (start 127 99.06) (end 127 104.14) (width 0.5) (layer B.Cu) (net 4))
 (segment (start 129.54 99.06) (end 129.54 104.14) (width 0.5) (layer B.Cu) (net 5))
 (segment (start 132.08 99.06) (end 132.08 104.14) (width 0.5) (layer B.Cu) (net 6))
 (segment (start 134.62 99.06) (end 134.62 104.14) (width 0.5) (layer B.Cu) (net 7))
 (segment (start 137.16 99.06) (end 137.16 104.14) (width 0.5) (layer B.Cu) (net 8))
 (segment (start 139.7 99.06) (end 139.7 104.14) (width 0.5) (layer B.Cu) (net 9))
 (segment (start 142.24 99.06) (end 142.24 104.14) (width 0.5) (layer B.Cu) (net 10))
 (segment (start 144.78 99.06) (end 144.78 104.14) (width 0.5) (layer B.Cu) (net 11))
 (segment (start 147.32 83.82) (end 147.32 95.25) (width 0.5) (layer F.Cu) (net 12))
 (segment (start 146.05 101.6) (end 147.32 104.14) (width 0.5) (layer F.Cu) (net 12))
 (segment (start 146.05 96.52) (end 146.05 101.6) (width 0.5) (layer F.Cu) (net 12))
 (segment (start 147.32 95.25) (end 146.05 96.52) (width 0.5) (layer F.Cu) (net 12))
 (segment (start 146.05 96.52) (end 146.05 96.52) (width 0.25) (layer F.Cu) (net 12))
 (segment (start 144.78 83.82) (end 144.78 93.98) (width 0.5) (layer F.Cu) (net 13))
 (segment (start 149.86 99.06) (end 149.86 104.14) (width 0.5) (layer B.Cu) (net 13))
 (segment (start 144.78 93.98) (end 149.86 99.06) (width 0.5) (layer B.Cu) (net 13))
 (via (at 144.78 93.98) (size 0.6) (drill 0.4) (layers F.Cu B.Cu) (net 13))
 (segment (start 152.4 104.14) (end 152.4 99.06) (width 0.5) (layer B.Cu) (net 14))
 (segment (start 142.24 91.44) (end 142.24 83.82) (width 0.5) (layer F.Cu) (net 14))
 (via (at 142.24 91.44) (size 0.6) (drill 0.4) (layers F.Cu B.Cu) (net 14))
 (segment (start 144.78 91.44) (end 142.24 91.44) (width 0.5) (layer B.Cu) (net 14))
 (segment (start 152.4 99.06) (end 144.78 91.44) (width 0.5) (layer B.Cu) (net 14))
 (segment (start 154.94 104.14) (end 154.94 99.06) (width 0.5) (layer B.Cu) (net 15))
 (segment (start 139.7 90.17) (end 139.7 83.82) (width 0.5) (layer F.Cu) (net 15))
 (via (at 139.7 90.17) (size 0.6) (drill 0.4) (layers F.Cu B.Cu) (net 15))
 (segment (start 146.05 90.17) (end 139.7 90.17) (width 0.5) (layer B.Cu) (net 15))
 (segment (start 154.94 99.06) (end 146.05 90.17) (width 0.5) (layer B.Cu) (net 15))
 (segment (start 157.48 104.14) (end 157.48 99.06) (width 0.5) (layer B.Cu) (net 16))
 (segment (start 142.24 88.9) (end 137.16 83.82) (width 0.5) (layer B.Cu) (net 16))
 (segment (start 147.32 88.9) (end 142.24 88.9) (width 0.5) (layer B.Cu) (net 16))
 (segment (start 157.48 99.06) (end 147.32 88.9) (width 0.5) (layer B.Cu) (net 16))
 (segment (start 142.24 80.01) (end 142.24 81.28) (width 0.5) (layer B.Cu) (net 17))
 (segment (start 162.56 101.6) (end 162.56 104.14) (width 0.5) (layer B.Cu) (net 17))
 (segment (start 148.59 87.63) (end 162.56 101.6) (width 0.5) (layer B.Cu) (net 17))
 (segment (start 146.05 87.63) (end 148.59 87.63) (width 0.5) (layer B.Cu) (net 17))
 (segment (start 143.51 85.09) (end 146.05 87.63) (width 0.5) (layer B.Cu) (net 17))
 (segment (start 143.51 82.55) (end 143.51 85.09) (width 0.5) (layer B.Cu) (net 17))
 (segment (start 142.24 81.28) (end 143.51 82.55) (width 0.5) (layer B.Cu) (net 17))
 (segment (start 142.24 76.2) (end 142.24 80.01) (width 0.5) (layer B.Cu) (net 17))
 (segment (start 144.78 80.01) (end 144.78 81.28) (width 0.5) (layer B.Cu) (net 18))
 (segment (start 165.1 101.6) (end 165.1 104.14) (width 0.5) (layer B.Cu) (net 18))
 (segment (start 149.86 86.36) (end 165.1 101.6) (width 0.5) (layer B.Cu) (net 18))
 (segment (start 147.32 86.36) (end 149.86 86.36) (width 0.5) (layer B.Cu) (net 18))
 (segment (start 146.05 85.09) (end 147.32 86.36) (width 0.5) (layer B.Cu) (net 18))
 (segment (start 146.05 82.55) (end 146.05 85.09) (width 0.5) (layer B.Cu) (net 18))
 (segment (start 144.78 81.28) (end 146.05 82.55) (width 0.5) (layer B.Cu) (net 18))
 (segment (start 144.78 76.2) (end 144.78 80.01) (width 0.5) (layer B.Cu) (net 18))
 (segment (start 147.32 80.01) (end 147.32 81.28) (width 0.5) (layer B.Cu) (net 19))
 (segment (start 167.64 101.6) (end 167.64 104.14) (width 0.5) (layer B.Cu) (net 19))
 (segment (start 147.32 81.28) (end 167.64 101.6) (width 0.5) (layer B.Cu) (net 19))
 (segment (start 147.32 76.2) (end 147.32 80.01) (width 0.5) (layer B.Cu) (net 19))
 (segment (start 149.86 80.01) (end 149.86 81.28) (width 0.5) (layer B.Cu) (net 20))
 (segment (start 170.18 101.6) (end 170.18 104.14) (width 0.5) (layer B.Cu) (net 20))
 (segment (start 149.86 81.28) (end 170.18 101.6) (width 0.5) (layer B.Cu) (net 20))
 (segment (start 149.86 76.2) (end 149.86 80.01) (width 0.5) (layer B.Cu) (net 20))
 (segment (start 152.4 80.01) (end 152.4 81.28) (width 0.5) (layer B.Cu) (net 21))
 (segment (start 172.72 101.6) (end 172.72 104.14) (width 0.5) (layer B.Cu) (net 21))
 (segment (start 152.4 81.28) (end 172.72 101.6) (width 0.5) (layer B.Cu) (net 21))
 (segment (start 152.4 76.2) (end 152.4 80.01) (width 0.5) (layer B.Cu) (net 21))
 (segment (start 154.94 80.01) (end 154.94 81.28) (width 0.5) (layer B.Cu) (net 22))
 (segment (start 175.26 101.6) (end 175.26 104.14) (width 0.5) (layer B.Cu) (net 22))
 (segment (start 154.94 81.28) (end 175.26 101.6) (width 0.5) (layer B.Cu) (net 22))
 (segment (start 154.94 76.2) (end 154.94 80.01) (width 0.5) (layer B.Cu) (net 22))
 (segment (start 157.48 80.01) (end 157.48 81.28) (width 0.5) (layer B.Cu) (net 23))
 (segment (start 177.8 101.6) (end 177.8 104.14) (width 0.5) (layer B.Cu) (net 23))
 (segment (start 157.48 81.28) (end 177.8 101.6) (width 0.5) (layer B.Cu) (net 23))
 (segment (start 157.48 76.2) (end 157.48 80.01) (width 0.5) (layer B.Cu) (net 23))
 (segment (start 160.02 80.01) (end 160.02 81.28) (width 0.5) (layer B.Cu) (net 24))
 (segment (start 180.34 101.6) (end 180.34 104.14) (width 0.5) (layer B.Cu) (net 24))
 (segment (start 160.02 81.28) (end 180.34 101.6) (width 0.5) (layer B.Cu) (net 24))
 (segment (start 160.02 76.2) (end 160.02 80.01) (width 0.5) (layer B.Cu) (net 24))
 (segment (start 118.11 68.58) (end 118.11 68.3895) (width 1) (layer B.Cu) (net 25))
 (segment (start 118.11 68.3895) (end 115.3795 65.659) (width 1) (layer B.Cu) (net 25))
 (segment (start 147.32 99.06) (end 144.78 96.52) (width 1) (layer B.Cu) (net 25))
 (segment (start 113.7285 65.659) (end 115.3795 65.659) (width 1) (layer B.Cu) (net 25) (status 10))
 (segment (start 140.97 96.52) (end 144.78 96.52) (width 1) (layer B.Cu) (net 25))
 (segment (start 134.62 90.17) (end 134.62 83.82) (width 1) (layer B.Cu) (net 25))
 (segment (start 134.62 90.17) (end 140.97 96.52) (width 1) (layer B.Cu) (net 25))
 (segment (start 118.11 68.58) (end 119.38 68.58) (width 1) (layer B.Cu) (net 25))
 (via (at 119.38 68.58) (size 0.6) (drill 0.4) (layers F.Cu B.Cu) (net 25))
 (segment (start 119.38 68.58) (end 119.38 76.2) (width 1) (layer F.Cu) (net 25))
 (segment (start 134.62 83.82) (end 132.08 83.82) (width 1) (layer B.Cu) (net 25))
 (segment (start 119.38 80.01) (end 119.38 81.28) (width 1) (layer B.Cu) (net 25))
 (segment (start 119.38 81.28) (end 120.65 82.55) (width 0.5) (layer B.Cu) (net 25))
 (segment (start 120.65 85.09) (end 121.92 86.36) (width 0.5) (layer B.Cu) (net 25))
 (segment (start 120.65 82.55) (end 120.65 85.09) (width 0.5) (layer B.Cu) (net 25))
 (segment (start 121.92 86.36) (end 130.81 86.36) (width 0.5) (layer B.Cu) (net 25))
 (segment (start 130.81 86.36) (end 132.08 85.09) (width 0.5) (layer B.Cu) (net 25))
 (segment (start 132.08 85.09) (end 132.08 83.82) (width 0.5) (layer B.Cu) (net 25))
 (segment (start 119.38 76.2) (end 119.38 80.01) (width 1) (layer B.Cu) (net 25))
 (segment (start 121.92 80.01) (end 121.92 83.82) (width 0.5) (layer B.Cu) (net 26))
 (segment (start 121.92 76.2) (end 121.92 80.01) (width 0.5) (layer B.Cu) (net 26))
 (segment (start 124.46 80.01) (end 124.46 83.82) (width 0.5) (layer B.Cu) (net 27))
 (segment (start 124.46 76.2) (end 124.46 80.01) (width 0.5) (layer B.Cu) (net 27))
 (segment (start 127 80.01) (end 127 83.82) (width 0.5) (layer B.Cu) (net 28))
 (segment (start 127 76.2) (end 127 80.01) (width 0.5) (layer B.Cu) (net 28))
 (segment (start 129.54 80.01) (end 129.54 83.82) (width 0.5) (layer B.Cu) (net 29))
 (segment (start 129.54 76.2) (end 129.54 80.01) (width 0.5) (layer B.Cu) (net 29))
 (segment (start 132.08 76.2) (end 132.08 80.01) (width 0.5) (layer B.Cu) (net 30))
 (segment (start 134.62 76.2) (end 134.62 80.01) (width 0.5) (layer B.Cu) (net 31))
 (segment (start 137.16 76.2) (end 137.16 80.01) (width 0.5) (layer B.Cu) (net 32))
 (segment (start 139.7 76.2) (end 139.7 80.01) (width 0.5) (layer B.Cu) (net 33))
 (segment (start 162.56 76.2) (end 162.56 80.01) (width 0.5) (layer B.Cu) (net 34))
 (segment (start 165.1 76.2) (end 165.1 80.01) (width 0.5) (layer B.Cu) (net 35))
 (segment (start 116.332 71.9455) (end 116.5225 71.9455) (width 1) (layer B.Cu) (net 36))
 (segment (start 116.5225 71.9455) (end 117.348 71.12) (width 1) (layer B.Cu) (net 36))
 (segment (start 118.0465 71.12) (end 117.348 71.12) (width 1) (layer B.Cu) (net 36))
 (segment (start 117.348 71.12) (end 115.5065 71.12) (width 1) (layer B.Cu) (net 36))
 (segment (start 115.5065 71.12) (end 114.935 70.5485) (width 1) (layer B.Cu) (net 36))
 (segment (start 116.84 72.4535) (end 117.9195 71.374) (width 1) (layer B.Cu) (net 36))
 (segment (start 118.0465 71.12) (end 119.38 71.12) (width 1) (layer B.Cu) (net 36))
 (segment (start 117.9195 71.247) (end 118.0465 71.12) (width 1) (layer B.Cu) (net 36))
 (segment (start 117.9195 71.374) (end 117.9195 71.247) (width 1) (layer B.Cu) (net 36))
 (segment (start 116.84 73.66) (end 116.84 72.4535) (width 1) (layer B.Cu) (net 36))
 (segment (start 116.84 72.4535) (end 116.332 71.9455) (width 1) (layer B.Cu) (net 36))
 (segment (start 116.332 71.9455) (end 114.935 70.5485) (width 1) (layer B.Cu) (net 36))
 (segment (start 114.935 70.5485) (end 114.1095 69.723) (width 1) (layer B.Cu) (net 36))
 (segment (start 113.7285 69.342) (end 113.7285 68.199) (width 1) (layer B.Cu) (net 36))
 (segment (start 114.1095 69.723) (end 113.7285 69.342) (width 1) (layer B.Cu) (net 36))
 (segment (start 167.64 76.2) (end 167.64 72.39) (width 1) (layer B.Cu) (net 36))
 (segment (start 166.37 71.12) (end 119.38 71.12) (width 1) (layer B.Cu) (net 36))
 (segment (start 167.64 72.39) (end 166.37 71.12) (width 1) (layer B.Cu) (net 36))
 (segment (start 119.38 71.12) (end 116.84 73.66) (width 1) (layer B.Cu) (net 36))
 (segment (start 116.84 81.28) (end 119.38 83.82) (width 1) (layer B.Cu) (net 36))
 (segment (start 116.84 73.66) (end 116.84 81.28) (width 1) (layer B.Cu) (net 36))
 (segment (start 167.64 76.2) (end 167.64 80.01) (width 1) (layer B.Cu) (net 36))
 (segment (start 167.64 60.96) (end 167.64 64.77) (width 0.5) (layer B.Cu) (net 37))
 (segment (start 165.1 60.96) (end 165.1 64.77) (width 0.5) (layer B.Cu) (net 38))
 (segment (start 162.56 60.96) (end 162.56 64.77) (width 0.5) (layer B.Cu) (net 39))
 (segment (start 160.02 60.96) (end 160.02 64.77) (width 0.5) (layer B.Cu) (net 40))
 (segment (start 157.48 60.96) (end 157.48 64.77) (width 0.5) (layer B.Cu) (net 41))
 (segment (start 154.94 60.96) (end 154.94 64.77) (width 0.5) (layer B.Cu) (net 42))
 (segment (start 152.4 60.96) (end 152.4 64.77) (width 0.5) (layer B.Cu) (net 43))
 (segment (start 149.86 60.96) (end 149.86 64.77) (width 0.5) (layer B.Cu) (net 44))
 (segment (start 147.32 60.96) (end 147.32 64.77) (width 0.5) (layer B.Cu) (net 45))
 (segment (start 144.78 60.96) (end 144.78 64.77) (width 0.5) (layer B.Cu) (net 46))
 (segment (start 142.24 60.96) (end 142.24 64.77) (width 0.5) (layer B.Cu) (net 47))
 (segment (start 139.7 60.96) (end 139.7 64.77) (width 0.5) (layer B.Cu) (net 48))
 (segment (start 137.16 60.96) (end 137.16 64.77) (width 0.5) (layer B.Cu) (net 49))
 (segment (start 134.62 60.96) (end 134.62 64.77) (width 0.5) (layer B.Cu) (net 50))
 (segment (start 132.08 60.96) (end 132.08 64.77) (width 0.5) (layer B.Cu) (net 51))
 (segment (start 129.54 60.96) (end 129.54 64.77) (width 0.5) (layer B.Cu) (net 52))
 (segment (start 127 60.96) (end 127 64.77) (width 0.5) (layer B.Cu) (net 53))
 (segment (start 124.46 60.96) (end 124.46 64.77) (width 0.5) (layer B.Cu) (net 54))
 (segment (start 121.92 60.96) (end 121.92 64.77) (width 0.5) (layer B.Cu) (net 55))
 (segment (start 119.38 60.96) (end 119.38 64.77) (width 0.5) (layer B.Cu) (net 56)))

